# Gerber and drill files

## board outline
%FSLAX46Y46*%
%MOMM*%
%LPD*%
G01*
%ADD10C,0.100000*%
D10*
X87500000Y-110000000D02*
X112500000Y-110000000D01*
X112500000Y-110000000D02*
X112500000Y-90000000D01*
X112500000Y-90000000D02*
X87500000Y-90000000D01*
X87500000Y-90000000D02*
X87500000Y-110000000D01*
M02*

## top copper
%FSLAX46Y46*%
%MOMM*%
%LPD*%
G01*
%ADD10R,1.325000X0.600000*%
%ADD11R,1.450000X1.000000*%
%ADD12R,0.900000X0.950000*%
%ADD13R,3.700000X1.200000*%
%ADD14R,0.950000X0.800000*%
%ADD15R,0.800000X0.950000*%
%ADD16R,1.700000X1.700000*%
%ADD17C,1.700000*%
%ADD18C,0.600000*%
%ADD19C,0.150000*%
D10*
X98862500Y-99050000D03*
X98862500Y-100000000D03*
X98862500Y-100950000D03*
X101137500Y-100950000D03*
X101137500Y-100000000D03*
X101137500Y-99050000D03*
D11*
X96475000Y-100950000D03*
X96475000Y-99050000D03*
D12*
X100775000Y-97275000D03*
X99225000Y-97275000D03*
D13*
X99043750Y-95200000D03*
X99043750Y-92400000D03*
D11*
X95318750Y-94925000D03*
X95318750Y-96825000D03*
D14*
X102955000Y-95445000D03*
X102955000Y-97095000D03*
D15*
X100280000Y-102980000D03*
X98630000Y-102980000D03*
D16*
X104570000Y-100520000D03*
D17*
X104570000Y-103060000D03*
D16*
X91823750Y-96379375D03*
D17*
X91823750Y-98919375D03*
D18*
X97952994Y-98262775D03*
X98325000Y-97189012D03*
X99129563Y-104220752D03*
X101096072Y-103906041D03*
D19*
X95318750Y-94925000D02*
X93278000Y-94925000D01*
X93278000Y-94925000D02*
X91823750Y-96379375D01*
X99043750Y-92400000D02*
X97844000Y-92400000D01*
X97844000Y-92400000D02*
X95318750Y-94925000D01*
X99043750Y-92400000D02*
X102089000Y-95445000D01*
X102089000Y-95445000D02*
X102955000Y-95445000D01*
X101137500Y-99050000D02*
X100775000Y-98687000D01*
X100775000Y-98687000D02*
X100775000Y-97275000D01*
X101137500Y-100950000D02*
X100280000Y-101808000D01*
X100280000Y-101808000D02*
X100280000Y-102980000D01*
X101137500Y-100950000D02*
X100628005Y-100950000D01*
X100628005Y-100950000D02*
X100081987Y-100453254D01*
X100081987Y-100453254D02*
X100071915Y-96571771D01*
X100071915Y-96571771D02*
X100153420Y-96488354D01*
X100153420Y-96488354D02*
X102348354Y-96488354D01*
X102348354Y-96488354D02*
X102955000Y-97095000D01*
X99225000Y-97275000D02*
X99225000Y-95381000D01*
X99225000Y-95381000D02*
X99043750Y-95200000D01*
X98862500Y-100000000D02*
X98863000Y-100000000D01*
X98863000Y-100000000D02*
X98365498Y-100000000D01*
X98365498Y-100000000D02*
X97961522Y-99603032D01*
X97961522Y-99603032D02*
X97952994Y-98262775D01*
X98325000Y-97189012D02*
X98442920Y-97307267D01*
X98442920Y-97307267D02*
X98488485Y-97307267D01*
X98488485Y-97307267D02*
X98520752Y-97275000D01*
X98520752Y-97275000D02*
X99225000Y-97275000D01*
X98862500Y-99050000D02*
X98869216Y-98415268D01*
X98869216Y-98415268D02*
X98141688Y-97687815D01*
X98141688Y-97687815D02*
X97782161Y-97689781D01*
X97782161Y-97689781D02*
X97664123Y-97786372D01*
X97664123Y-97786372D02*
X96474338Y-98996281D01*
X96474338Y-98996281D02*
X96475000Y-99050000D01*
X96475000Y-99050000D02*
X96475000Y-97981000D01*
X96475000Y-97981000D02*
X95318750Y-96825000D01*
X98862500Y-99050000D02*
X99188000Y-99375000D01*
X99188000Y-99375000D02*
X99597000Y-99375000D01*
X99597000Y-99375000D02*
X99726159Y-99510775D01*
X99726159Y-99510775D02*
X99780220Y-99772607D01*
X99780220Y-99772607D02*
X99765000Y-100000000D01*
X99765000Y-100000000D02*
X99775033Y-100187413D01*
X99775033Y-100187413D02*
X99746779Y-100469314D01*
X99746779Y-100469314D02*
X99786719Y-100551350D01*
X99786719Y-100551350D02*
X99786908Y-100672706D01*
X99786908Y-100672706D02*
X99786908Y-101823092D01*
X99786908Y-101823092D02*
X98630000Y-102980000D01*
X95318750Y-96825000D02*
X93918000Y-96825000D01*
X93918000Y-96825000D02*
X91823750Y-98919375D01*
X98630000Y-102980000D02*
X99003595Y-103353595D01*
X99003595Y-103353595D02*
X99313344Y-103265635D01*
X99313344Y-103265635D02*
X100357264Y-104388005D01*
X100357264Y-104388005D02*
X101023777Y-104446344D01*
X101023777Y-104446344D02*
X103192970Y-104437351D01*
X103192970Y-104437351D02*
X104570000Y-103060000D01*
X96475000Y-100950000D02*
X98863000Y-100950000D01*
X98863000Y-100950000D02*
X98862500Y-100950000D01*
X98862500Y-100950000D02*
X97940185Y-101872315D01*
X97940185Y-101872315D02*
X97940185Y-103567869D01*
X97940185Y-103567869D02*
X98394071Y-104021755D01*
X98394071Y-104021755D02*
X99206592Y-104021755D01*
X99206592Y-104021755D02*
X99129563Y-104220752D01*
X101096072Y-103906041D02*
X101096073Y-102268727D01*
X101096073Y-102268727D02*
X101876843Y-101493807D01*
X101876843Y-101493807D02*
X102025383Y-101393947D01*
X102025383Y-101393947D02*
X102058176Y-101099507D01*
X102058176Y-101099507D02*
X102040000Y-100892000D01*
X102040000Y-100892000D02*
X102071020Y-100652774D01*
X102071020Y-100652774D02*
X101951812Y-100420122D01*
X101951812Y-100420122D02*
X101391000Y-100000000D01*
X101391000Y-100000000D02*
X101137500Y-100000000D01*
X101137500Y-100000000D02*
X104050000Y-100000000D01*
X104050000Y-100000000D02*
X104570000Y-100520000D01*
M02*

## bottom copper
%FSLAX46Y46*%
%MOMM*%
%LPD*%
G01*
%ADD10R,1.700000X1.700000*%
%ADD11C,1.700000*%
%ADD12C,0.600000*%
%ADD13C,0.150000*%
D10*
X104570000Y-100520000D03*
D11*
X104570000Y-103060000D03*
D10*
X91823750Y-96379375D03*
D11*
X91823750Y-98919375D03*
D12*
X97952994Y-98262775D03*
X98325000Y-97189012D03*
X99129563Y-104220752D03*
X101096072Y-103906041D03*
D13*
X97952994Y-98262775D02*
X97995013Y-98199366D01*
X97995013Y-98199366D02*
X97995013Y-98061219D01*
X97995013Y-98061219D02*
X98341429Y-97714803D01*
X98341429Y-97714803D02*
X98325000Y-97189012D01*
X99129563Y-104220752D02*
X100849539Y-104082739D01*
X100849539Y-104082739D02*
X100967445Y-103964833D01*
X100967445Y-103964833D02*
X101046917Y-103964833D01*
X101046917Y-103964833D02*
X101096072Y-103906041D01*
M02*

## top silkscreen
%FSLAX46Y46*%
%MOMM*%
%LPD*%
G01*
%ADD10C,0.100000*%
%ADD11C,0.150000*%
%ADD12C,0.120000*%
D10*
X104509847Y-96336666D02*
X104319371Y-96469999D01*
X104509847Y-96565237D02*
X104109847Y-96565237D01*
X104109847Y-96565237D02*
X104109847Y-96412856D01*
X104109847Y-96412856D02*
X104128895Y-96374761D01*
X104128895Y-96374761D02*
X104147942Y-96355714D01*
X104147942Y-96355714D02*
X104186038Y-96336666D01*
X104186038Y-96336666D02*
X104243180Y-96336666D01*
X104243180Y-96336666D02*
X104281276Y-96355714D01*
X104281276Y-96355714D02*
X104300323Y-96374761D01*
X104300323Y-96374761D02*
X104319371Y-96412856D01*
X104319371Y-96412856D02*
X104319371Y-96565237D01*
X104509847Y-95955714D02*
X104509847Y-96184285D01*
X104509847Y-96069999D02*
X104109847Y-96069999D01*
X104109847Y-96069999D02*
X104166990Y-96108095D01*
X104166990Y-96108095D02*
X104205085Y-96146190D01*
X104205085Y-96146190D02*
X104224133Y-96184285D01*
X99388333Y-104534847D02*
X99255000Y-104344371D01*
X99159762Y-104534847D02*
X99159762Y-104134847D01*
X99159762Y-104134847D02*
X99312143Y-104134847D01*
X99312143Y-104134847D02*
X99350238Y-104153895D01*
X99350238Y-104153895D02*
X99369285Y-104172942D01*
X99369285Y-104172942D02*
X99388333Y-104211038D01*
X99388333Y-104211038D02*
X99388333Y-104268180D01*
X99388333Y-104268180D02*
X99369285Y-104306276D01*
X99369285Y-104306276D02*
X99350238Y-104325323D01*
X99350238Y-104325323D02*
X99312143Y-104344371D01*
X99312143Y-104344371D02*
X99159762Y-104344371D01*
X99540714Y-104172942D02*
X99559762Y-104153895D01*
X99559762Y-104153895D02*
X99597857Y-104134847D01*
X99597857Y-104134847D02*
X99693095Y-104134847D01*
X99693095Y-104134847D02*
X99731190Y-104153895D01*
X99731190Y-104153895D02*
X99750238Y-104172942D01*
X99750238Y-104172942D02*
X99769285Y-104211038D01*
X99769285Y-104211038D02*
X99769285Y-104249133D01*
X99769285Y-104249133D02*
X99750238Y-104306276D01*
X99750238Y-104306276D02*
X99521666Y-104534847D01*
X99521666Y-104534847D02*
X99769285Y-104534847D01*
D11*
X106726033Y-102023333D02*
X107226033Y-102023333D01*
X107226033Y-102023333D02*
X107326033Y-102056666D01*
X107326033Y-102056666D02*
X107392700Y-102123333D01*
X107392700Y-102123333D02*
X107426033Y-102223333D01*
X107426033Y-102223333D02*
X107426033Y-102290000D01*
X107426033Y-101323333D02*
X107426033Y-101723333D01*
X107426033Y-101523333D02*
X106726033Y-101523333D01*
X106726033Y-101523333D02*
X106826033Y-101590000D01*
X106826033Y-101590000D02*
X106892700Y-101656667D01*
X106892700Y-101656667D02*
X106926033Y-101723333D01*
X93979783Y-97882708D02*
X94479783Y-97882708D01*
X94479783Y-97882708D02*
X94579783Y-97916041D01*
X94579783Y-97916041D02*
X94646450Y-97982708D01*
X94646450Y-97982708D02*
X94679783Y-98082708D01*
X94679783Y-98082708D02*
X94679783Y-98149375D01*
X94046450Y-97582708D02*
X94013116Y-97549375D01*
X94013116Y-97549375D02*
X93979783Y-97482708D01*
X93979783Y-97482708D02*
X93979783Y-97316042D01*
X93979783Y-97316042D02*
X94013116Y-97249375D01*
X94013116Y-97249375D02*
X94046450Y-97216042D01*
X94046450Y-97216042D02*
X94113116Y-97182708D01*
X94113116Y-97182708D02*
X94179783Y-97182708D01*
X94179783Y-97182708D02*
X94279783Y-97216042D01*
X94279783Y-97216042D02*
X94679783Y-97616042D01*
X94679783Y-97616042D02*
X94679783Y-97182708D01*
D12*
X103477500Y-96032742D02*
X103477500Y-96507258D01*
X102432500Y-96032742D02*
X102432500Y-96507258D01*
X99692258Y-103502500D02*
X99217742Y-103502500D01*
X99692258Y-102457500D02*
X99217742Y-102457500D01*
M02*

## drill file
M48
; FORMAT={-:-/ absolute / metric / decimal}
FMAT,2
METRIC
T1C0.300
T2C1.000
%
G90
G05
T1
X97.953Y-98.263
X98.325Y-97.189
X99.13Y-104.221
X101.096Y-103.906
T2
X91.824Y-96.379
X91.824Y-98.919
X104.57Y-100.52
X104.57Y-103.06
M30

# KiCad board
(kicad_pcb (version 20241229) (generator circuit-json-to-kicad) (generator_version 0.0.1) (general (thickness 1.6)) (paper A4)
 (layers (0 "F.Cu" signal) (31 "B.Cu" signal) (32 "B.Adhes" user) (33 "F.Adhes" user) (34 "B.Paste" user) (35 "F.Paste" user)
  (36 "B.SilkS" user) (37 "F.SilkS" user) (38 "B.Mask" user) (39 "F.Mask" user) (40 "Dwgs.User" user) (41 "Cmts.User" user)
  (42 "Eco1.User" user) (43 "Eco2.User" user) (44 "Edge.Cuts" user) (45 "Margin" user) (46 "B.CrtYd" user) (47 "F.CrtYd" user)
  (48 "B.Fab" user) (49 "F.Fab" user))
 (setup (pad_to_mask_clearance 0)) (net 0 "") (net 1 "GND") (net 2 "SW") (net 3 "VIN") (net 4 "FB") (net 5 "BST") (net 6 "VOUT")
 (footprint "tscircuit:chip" (layer F.Cu) (at 100 100 0)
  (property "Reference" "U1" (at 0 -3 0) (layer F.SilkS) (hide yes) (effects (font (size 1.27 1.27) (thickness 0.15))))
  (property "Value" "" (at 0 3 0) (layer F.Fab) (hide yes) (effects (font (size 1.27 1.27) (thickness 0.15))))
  (pad "1" smd rect (at -1.1375 -0.95 0) (size 1.325 0.6) (layers F.Cu F.Mask) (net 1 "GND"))
  (pad "2" smd rect (at -1.1375 0 0) (size 1.325 0.6) (layers F.Cu F.Mask) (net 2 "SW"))
  (pad "3" smd rect (at -1.1375 0.95 0) (size 1.325 0.6) (layers F.Cu F.Mask) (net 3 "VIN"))
  (pad "4" smd rect (at 1.1375 0.95 0) (size 1.325 0.6) (layers F.Cu F.Mask) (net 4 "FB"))
  (pad "5" smd rect (at 1.1375 0 0) (size 1.325 0.6) (layers F.Cu F.Mask) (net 3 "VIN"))
  (pad "6" smd rect (at 1.1375 -0.95 0) (size 1.325 0.6) (layers F.Cu F.Mask) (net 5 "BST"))
  (pad "" smd rect (at -1.1375 -0.95 0) (size 0.9274999999999999 0.42) (layers F.Paste))
  (pad "" smd rect (at -1.1375 0 0) (size 0.9274999999999999 0.42) (layers F.Paste))
  (pad "" smd rect (at -1.1375 0.95 0) (size 0.9274999999999999 0.42) (layers F.Paste))
  (pad "" smd rect (at 1.1375 0.95 0) (size 0.9274999999999999 0.42) (layers F.Paste))
  (pad "" smd rect (at 1.1375 0 0) (size 0.9274999999999999 0.42) (layers F.Paste))
  (pad "" smd rect (at 1.1375 -0.95 0) (size 0.9274999999999999 0.42) (layers F.Paste)))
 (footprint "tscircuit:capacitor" (layer F.Cu) (at 96.475 100 90)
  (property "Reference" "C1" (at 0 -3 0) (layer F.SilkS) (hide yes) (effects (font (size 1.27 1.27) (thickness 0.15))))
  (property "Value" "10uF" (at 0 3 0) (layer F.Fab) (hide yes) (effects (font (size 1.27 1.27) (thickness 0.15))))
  (pad "1" smd rect (at -0.95 0 0) (size 1.45 1) (layers F.Cu F.Mask) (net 3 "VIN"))
  (pad "2" smd rect (at 0.95 0 0) (size 1.45 1) (layers F.Cu F.Mask) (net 1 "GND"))
  (pad "" smd rect (at -0.95 0 0) (size 1.015 0.7) (layers F.Paste))
  (pad "" smd rect (at 0.95 0 0) (size 1.015 0.7) (layers F.Paste)))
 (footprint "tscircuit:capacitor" (layer F.Cu) (at 100 97.275 180)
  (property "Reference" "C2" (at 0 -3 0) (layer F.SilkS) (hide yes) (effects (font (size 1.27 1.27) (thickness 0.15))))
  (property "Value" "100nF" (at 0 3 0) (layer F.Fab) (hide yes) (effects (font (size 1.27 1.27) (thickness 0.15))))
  (pad "1" smd rect (at -0.775 0 0) (size 0.9 0.95) (layers F.Cu F.Mask) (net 5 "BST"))
  (pad "2" smd rect (at 0.775 0 0) (size 0.9 0.95) (layers F.Cu F.Mask) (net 2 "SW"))
  (pad "" smd rect (at -0.775 0 0) (size 0.63 0.6649999999999999) (layers F.Paste))
  (pad "" smd rect (at 0.775 0 0) (size 0.63 0.6649999999999999) (layers F.Paste)))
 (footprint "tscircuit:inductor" (layer F.Cu) (at 99.04375 93.8 90)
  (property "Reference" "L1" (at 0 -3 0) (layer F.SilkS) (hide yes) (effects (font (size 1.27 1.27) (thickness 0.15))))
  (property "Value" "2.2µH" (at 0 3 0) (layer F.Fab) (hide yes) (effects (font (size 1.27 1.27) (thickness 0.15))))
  (pad "1" smd rect (at -1.3999999999999995 -1.1102230246251565e-16 0) (size 3.7 1.2) (layers F.Cu F.Mask) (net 2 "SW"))
  (pad "2" smd rect (at 1.3999999999999995 0 0) (size 3.7 1.2) (layers F.Cu F.Mask) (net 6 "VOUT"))
  (pad "" smd rect (at -1.3999999999999995 -1.1102230246251565e-16 0) (size 2.59 0.84) (layers F.Paste))
  (pad "" smd rect (at 1.3999999999999995 0 0) (size 2.59 0.84) (layers F.Paste)))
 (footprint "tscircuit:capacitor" (layer F.Cu) (at 95.31875 95.875 -90.00000000000001)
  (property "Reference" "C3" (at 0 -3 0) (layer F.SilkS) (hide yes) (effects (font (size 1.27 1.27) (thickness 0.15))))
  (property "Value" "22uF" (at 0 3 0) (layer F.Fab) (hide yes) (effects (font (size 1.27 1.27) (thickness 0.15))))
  (pad "1" smd rect (at -0.9500000000000002 0 0) (size 1.45 1) (layers F.Cu F.Mask) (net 6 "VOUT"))
  (pad "2" smd rect (at 0.9500000000000002 -8.881784197001252e-16 0) (size 1.45 1) (layers F.Cu F.Mask) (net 1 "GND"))
  (pad "" smd rect (at -0.9500000000000002 0 0) (size 1.015 0.7) (layers F.Paste))
  (pad "" smd rect (at 0.9500000000000002 -8.881784197001252e-16 0) (size 1.015 0.7) (layers F.Paste)))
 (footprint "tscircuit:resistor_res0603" (layer F.Cu) (at 102.955 96.27 -90.00000000000001)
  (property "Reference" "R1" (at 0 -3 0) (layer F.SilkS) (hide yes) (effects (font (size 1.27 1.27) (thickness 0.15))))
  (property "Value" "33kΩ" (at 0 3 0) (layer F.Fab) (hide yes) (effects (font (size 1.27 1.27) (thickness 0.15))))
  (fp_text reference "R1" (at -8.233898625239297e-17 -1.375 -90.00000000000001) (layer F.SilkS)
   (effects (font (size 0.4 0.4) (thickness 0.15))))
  (fp_line (start -0.23725799999999994 -0.5224999999999999) (end 0.237258 -0.5225000000000001) (stroke (width 0.12) (type default))
   (layer F.SilkS))
  (fp_line (start -0.237258 0.5225000000000001) (end 0.23725799999999994 0.5224999999999999) (stroke (width 0.12) (type default))
   (layer F.SilkS))
  (pad "1" smd rect (at -0.8249999999999997 4.440892098500626e-16 0) (size 0.95 0.8) (layers F.Cu F.Mask) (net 6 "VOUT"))
  (pad "2" smd rect (at 0.8250000000000002 0 0) (size 0.95 0.8) (layers F.Cu F.Mask) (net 4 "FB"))
  (pad "" smd rect (at -0.8249999999999997 4.440892098500626e-16 0) (size 0.6649999999999999 0.5599999999999999) (layers F.Paste))
  (pad "" smd rect (at 0.8250000000000002 0 0) (size 0.6649999999999999 0.5599999999999999) (layers F.Paste)))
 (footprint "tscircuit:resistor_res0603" (layer F.Cu) (at 99.455 102.98 180)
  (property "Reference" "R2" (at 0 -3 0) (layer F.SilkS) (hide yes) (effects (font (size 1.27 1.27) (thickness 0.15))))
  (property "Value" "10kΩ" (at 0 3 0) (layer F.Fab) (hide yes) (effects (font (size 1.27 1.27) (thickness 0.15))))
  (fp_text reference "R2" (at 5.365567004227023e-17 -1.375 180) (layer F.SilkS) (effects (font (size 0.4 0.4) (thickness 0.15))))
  (fp_line (start -0.23725800000000002 -0.5225) (end 0.23725800000000002 -0.5225) (stroke (width 0.12) (type default)) (layer F.SilkS))
  (fp_line (start -0.23725800000000002 0.5225) (end 0.23725800000000002 0.5225) (stroke (width 0.12) (type default)) (layer F.SilkS))
  (pad "1" smd rect (at -0.825 0 0) (size 0.8 0.95) (layers F.Cu F.Mask) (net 4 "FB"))
  (pad "2" smd rect (at 0.8249999999999998 0 0) (size 0.8 0.95) (layers F.Cu F.Mask) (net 1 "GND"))
  (pad "" smd rect (at -0.825 0 0) (size 0.5599999999999999 0.6649999999999999) (layers F.Paste))
  (pad "" smd rect (at 0.8249999999999998 0 0) (size 0.5599999999999999 0.6649999999999999) (layers F.Paste)))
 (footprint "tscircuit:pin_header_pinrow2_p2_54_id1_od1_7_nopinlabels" (layer F.Cu) (at 104.57 101.79 -90.00000000000001)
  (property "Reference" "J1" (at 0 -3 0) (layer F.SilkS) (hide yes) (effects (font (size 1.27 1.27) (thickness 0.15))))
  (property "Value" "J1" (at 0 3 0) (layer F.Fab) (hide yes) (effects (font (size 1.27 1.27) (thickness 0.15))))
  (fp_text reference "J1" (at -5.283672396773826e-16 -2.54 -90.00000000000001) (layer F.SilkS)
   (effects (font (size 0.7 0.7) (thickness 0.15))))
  (pad "1" thru_hole rect (at -1.27 4.862282247637226e-16 270) (size 1.7 1.7) (drill 1) (layers *.Cu *.Mask) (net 3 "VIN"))
  (pad "2" thru_hole circle (at 1.27 -4.862282247637226e-16 0) (size 1.7 1.7) (drill 1) (layers *.Cu *.Mask) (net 1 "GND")))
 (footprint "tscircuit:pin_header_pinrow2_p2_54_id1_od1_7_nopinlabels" (layer F.Cu) (at 91.82375 97.649375 -90.00000000000001)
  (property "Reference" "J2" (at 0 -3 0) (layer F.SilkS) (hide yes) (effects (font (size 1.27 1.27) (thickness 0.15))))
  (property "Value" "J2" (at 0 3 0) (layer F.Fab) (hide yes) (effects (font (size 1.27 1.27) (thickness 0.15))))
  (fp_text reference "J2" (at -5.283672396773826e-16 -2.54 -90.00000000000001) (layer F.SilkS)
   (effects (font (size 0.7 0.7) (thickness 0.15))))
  (pad "1" thru_hole rect (at -1.27 4.862282247637226e-16 270) (size 1.7 1.7) (drill 1) (layers *.Cu *.Mask) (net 6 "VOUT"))
  (pad "2" thru_hole circle (at 1.27 -4.862282247637226e-16 0) (size 1.7 1.7) (drill 1) (layers *.Cu *.Mask) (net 1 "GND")))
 (segment (start 95.31875 94.925) (end 93.278 94.925) (width 0.15) (layer F.Cu) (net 6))
 (segment (start 93.278 94.925) (end 91.82375 96.379375) (width 0.15) (layer F.Cu) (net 6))
 (segment (start 99.04375 92.4) (end 97.844 92.4) (width 0.15) (layer F.Cu) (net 6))
 (segment (start 97.844 92.4) (end 95.31875 94.925) (width 0.15) (layer F.Cu) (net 6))
 (segment (start 99.04375 92.4) (end 102.089 95.445) (width 0.15) (layer F.Cu) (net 6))
 (segment (start 102.089 95.445) (end 102.955 95.445) (width 0.15) (layer F.Cu) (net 6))
 (segment (start 101.1375 99.05) (end 100.775 98.687) (width 0.15) (layer F.Cu) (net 5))
 (segment (start 100.775 98.687) (end 100.775 97.275) (width 0.15) (layer F.Cu) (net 5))
 (segment (start 101.1375 100.95) (end 100.28 101.808) (width 0.15) (layer F.Cu) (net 4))
 (segment (start 100.28 101.808) (end 100.28 102.98) (width 0.15) (layer F.Cu) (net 4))
 (segment (start 101.1375 100.95) (end 100.62800530420733 100.95) (width 0.15) (layer F.Cu) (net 4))
 (segment (start 100.62800530420733 100.95) (end 100.08198698397962 100.45325403035147) (width 0.15) (layer F.Cu) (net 4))
 (segment (start 100.08198698397962 100.45325403035147) (end 100.07191484380009 96.57177142896099) (width 0.15) (layer F.Cu) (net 4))
 (segment (start 100.07191484380009 96.57177142896099) (end 100.15342021494793 96.48835356198515) (width 0.15) (layer F.Cu) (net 4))
 (segment (start 100.15342021494793 96.48835356198515) (end 102.34835356198515 96.48835356198515) (width 0.15) (layer F.Cu) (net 4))
 (segment (start 102.34835356198515 96.48835356198515) (end 102.955 97.095) (width 0.15) (layer F.Cu) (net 4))
 (segment (start 99.225 97.275) (end 99.225 95.381) (width 0.15) (layer F.Cu) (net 2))
 (segment (start 99.225 95.381) (end 99.04375 95.2) (width 0.15) (layer F.Cu) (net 2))
 (segment (start 98.8625 100) (end 98.863 100) (width 0.15) (layer F.Cu) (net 2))
 (segment (start 98.863 100) (end 98.36549796688661 100) (width 0.15) (layer F.Cu) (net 2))
 (segment (start 98.36549796688661 100) (end 97.96152206184571 99.60303247482807) (width 0.15) (layer F.Cu) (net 2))
 (segment (start 97.96152206184571 99.60303247482807) (end 97.95299373907991 98.26277506287174) (width 0.15) (layer F.Cu) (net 2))
 (segment (start 97.95299373907991 98.26277506287174) (end 97.99501342727841 98.19936617827366) (width 0.15) (layer B.Cu) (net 2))
 (segment (start 97.99501342727841 98.19936617827366) (end 97.99501342727841 98.06121850387677) (width 0.15) (layer B.Cu) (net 2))
 (segment (start 97.99501342727841 98.06121850387677) (end 98.34142863944501 97.71480329171017) (width 0.15) (layer B.Cu) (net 2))
 (segment (start 98.34142863944501 97.71480329171017) (end 98.325 97.18901219470303) (width 0.15) (layer B.Cu) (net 2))
 (segment (start 98.325 97.18901219470303) (end 98.44292027198014 97.30726702794956) (width 0.15) (layer F.Cu) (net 2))
 (segment (start 98.44292027198014 97.30726702794956) (end 98.48848502187742 97.30726702794956) (width 0.15) (layer F.Cu) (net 2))
 (segment (start 98.48848502187742 97.30726702794956) (end 98.52075204982698 97.275) (width 0.15) (layer F.Cu) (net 2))
 (segment (start 98.52075204982698 97.275) (end 99.225 97.275) (width 0.15) (layer F.Cu) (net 2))
 (segment (start 98.8625 99.05) (end 98.86921649402048 98.41526766341771) (width 0.15) (layer F.Cu) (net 1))
 (segment (start 98.86921649402048 98.41526766341771) (end 98.14168757311079 97.68781511530996) (width 0.15) (layer F.Cu) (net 1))
 (segment (start 98.14168757311079 97.68781511530996) (end 97.78216063400573 97.68978081419841) (width 0.15) (layer F.Cu) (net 1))
 (segment (start 97.78216063400573 97.68978081419841) (end 97.66412276517964 97.78637179095722) (width 0.15) (layer F.Cu) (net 1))
 (segment (start 97.66412276517964 97.78637179095722) (end 96.47433845386279 98.99628114309799) (width 0.15) (layer F.Cu) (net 1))
 (segment (start 96.47433845386279 98.99628114309799) (end 96.475 99.05) (width 0.15) (layer F.Cu) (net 1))
 (segment (start 96.475 99.05) (end 96.475 97.981) (width 0.15) (layer F.Cu) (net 1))
 (segment (start 96.475 97.981) (end 95.31875 96.825) (width 0.15) (layer F.Cu) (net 1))
 (segment (start 98.8625 99.05) (end 99.188 99.375) (width 0.15) (layer F.Cu) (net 1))
 (segment (start 99.188 99.375) (end 99.597 99.375) (width 0.15) (layer F.Cu) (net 1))
 (segment (start 99.597 99.375) (end 99.72615868378477 99.51077535921002) (width 0.15) (layer F.Cu) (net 1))
 (segment (start 99.72615868378477 99.51077535921002) (end 99.78021974833956 99.77260683791522) (width 0.15) (layer F.Cu) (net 1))
 (segment (start 99.78021974833956 99.77260683791522) (end 99.765 100) (width 0.15) (layer F.Cu) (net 1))
 (segment (start 99.765 100) (end 99.77503340590779 100.18741348705161) (width 0.15) (layer F.Cu) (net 1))
 (segment (start 99.77503340590779 100.18741348705161) (end 99.74677949552942 100.46931385755846) (width 0.15) (layer F.Cu) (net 1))
 (segment (start 99.74677949552942 100.46931385755846) (end 99.78671880582407 100.55134963395433) (width 0.15) (layer F.Cu) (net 1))
 (segment (start 99.78671880582407 100.55134963395433) (end 99.78690846742921 100.67270577179946) (width 0.15) (layer F.Cu) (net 1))
 (segment (start 99.78690846742921 100.67270577179946) (end 99.78690846742921 101.82309153257079) (width 0.15) (layer F.Cu) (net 1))
 (segment (start 99.78690846742921 101.82309153257079) (end 98.63 102.98) (width 0.15) (layer F.Cu) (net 1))
 (segment (start 95.31875 96.825) (end 93.918 96.825) (width 0.15) (layer F.Cu) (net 1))
 (segment (start 93.918 96.825) (end 91.82375 98.919375) (width 0.15) (layer F.Cu) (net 1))
 (segment (start 98.63 102.98) (end 99.00359542347563 103.35359542347562) (width 0.15) (layer F.Cu) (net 1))
 (segment (start 99.00359542347563 103.35359542347562) (end 99.31334367499444 103.26563512603619) (width 0.15) (layer F.Cu) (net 1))
 (segment (start 99.31334367499444 103.26563512603619) (end 100.35726391937054 104.38800469974399) (width 0.15) (layer F.Cu) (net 1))
 (segment (start 100.35726391937054 104.38800469974399) (end 101.0237766795221 104.44634428796458) (width 0.15) (layer F.Cu) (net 1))
 (segment (start 101.0237766795221 104.44634428796458) (end 103.19297011969174 104.43735104489525) (width 0.15) (layer F.Cu) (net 1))
 (segment (start 103.19297011969174 104.43735104489525) (end 104.57 103.06) (width 0.15) (layer F.Cu) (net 1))
 (segment (start 96.475 100.95) (end 98.863 100.95) (width 0.15) (layer F.Cu) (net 3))
 (segment (start 98.863 100.95) (end 98.8625 100.95) (width 0.15) (layer F.Cu) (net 3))
 (segment (start 98.8625 100.95) (end 97.94018506917263 101.87231493082737) (width 0.15) (layer F.Cu) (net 3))
 (segment (start 97.94018506917263 101.87231493082737) (end 97.94018506917263 103.56786892787946) (width 0.15) (layer F.Cu) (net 3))
 (segment (start 97.94018506917263 103.56786892787946) (end 98.39407070624574 104.02175456495257) (width 0.15) (layer F.Cu) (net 3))
 (segment (start 98.39407070624574 104.02175456495257) (end 99.20659193717259 104.02175456495257) (width 0.15) (layer F.Cu) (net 3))
 (segment (start 99.20659193717259 104.02175456495257) (end 99.12956253239899 104.22075201675698) (width 0.15) (layer F.Cu) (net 3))
 (segment (start 99.12956253239899 104.22075201675698) (end 100.84953929056475 104.08273858846798) (width 0.15) (layer B.Cu) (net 3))
 (segment (start 100.84953929056475 104.08273858846798) (end 100.96744489109214 103.96483298794057) (width 0.15) (layer B.Cu) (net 3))
 (segment (start 100.96744489109214 103.96483298794057) (end 101.04691662014254 103.96483298794057) (width 0.15) (layer B.Cu) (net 3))
 (segment (start 101.04691662014254 103.96483298794057) (end 101.09607192297246 103.90604059630047) (width 0.15) (layer B.Cu) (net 3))
 (segment (start 101.09607192297246 103.90604059630047) (end 101.09607317819663 102.26872662957757) (width 0.15) (layer F.Cu) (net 3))
 (segment (start 101.09607317819663 102.26872662957757) (end 101.8768430110914 101.49380659976742) (width 0.15) (layer F.Cu) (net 3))
 (segment (start 101.8768430110914 101.49380659976742) (end 102.02538271553946 101.3939466344558) (width 0.15) (layer F.Cu) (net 3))
 (segment (start 102.02538271553946 101.3939466344558) (end 102.0581758931019 101.09950713435208) (width 0.15) (layer F.Cu) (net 3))
 (segment (start 102.0581758931019 101.09950713435208) (end 102.04 100.892) (width 0.15) (layer F.Cu) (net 3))
 (segment (start 102.04 100.892) (end 102.07102013225118 100.65277358134622) (width 0.15) (layer F.Cu) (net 3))
 (segment (start 102.07102013225118 100.65277358134622) (end 101.95181219517089 100.4201216714162) (width 0.15) (layer F.Cu) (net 3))
 (segment (start 101.95181219517089 100.4201216714162) (end 101.391 100) (width 0.15) (layer F.Cu) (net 3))
 (segment (start 101.391 100) (end 101.1375 100) (width 0.15) (layer F.Cu) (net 3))
 (segment (start 101.1375 100) (end 104.05 100) (width 0.15) (layer F.Cu) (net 3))
 (segment (start 104.05 100) (end 104.57 100.52) (width 0.15) (layer F.Cu) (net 3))
 (gr_line (start 87.5 110) (end 112.5 110) (width 0.1) (layer Edge.Cuts))
 (gr_line (start 112.5 110) (end 112.5 90) (width 0.1) (layer Edge.Cuts))
 (gr_line (start 112.5 90) (end 87.5 90) (width 0.1) (layer Edge.Cuts))
 (gr_line (start 87.5 90) (end 87.5 110) (width 0.1) (layer Edge.Cuts))
 (via (at 97.95299373907991 98.26277506287174) (size 0.6) (drill 0.3) (layers F.Cu B.Cu) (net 2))
 (via (at 98.325 97.18901219470303) (size 0.6) (drill 0.3) (layers F.Cu B.Cu) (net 2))
 (via (at 99.12956253239899 104.22075201675698) (size 0.6) (drill 0.3) (layers F.Cu B.Cu) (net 3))
 (via (at 101.09607192297246 103.90604059630047) (size 0.6) (drill 0.3) (layers F.Cu B.Cu) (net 3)))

